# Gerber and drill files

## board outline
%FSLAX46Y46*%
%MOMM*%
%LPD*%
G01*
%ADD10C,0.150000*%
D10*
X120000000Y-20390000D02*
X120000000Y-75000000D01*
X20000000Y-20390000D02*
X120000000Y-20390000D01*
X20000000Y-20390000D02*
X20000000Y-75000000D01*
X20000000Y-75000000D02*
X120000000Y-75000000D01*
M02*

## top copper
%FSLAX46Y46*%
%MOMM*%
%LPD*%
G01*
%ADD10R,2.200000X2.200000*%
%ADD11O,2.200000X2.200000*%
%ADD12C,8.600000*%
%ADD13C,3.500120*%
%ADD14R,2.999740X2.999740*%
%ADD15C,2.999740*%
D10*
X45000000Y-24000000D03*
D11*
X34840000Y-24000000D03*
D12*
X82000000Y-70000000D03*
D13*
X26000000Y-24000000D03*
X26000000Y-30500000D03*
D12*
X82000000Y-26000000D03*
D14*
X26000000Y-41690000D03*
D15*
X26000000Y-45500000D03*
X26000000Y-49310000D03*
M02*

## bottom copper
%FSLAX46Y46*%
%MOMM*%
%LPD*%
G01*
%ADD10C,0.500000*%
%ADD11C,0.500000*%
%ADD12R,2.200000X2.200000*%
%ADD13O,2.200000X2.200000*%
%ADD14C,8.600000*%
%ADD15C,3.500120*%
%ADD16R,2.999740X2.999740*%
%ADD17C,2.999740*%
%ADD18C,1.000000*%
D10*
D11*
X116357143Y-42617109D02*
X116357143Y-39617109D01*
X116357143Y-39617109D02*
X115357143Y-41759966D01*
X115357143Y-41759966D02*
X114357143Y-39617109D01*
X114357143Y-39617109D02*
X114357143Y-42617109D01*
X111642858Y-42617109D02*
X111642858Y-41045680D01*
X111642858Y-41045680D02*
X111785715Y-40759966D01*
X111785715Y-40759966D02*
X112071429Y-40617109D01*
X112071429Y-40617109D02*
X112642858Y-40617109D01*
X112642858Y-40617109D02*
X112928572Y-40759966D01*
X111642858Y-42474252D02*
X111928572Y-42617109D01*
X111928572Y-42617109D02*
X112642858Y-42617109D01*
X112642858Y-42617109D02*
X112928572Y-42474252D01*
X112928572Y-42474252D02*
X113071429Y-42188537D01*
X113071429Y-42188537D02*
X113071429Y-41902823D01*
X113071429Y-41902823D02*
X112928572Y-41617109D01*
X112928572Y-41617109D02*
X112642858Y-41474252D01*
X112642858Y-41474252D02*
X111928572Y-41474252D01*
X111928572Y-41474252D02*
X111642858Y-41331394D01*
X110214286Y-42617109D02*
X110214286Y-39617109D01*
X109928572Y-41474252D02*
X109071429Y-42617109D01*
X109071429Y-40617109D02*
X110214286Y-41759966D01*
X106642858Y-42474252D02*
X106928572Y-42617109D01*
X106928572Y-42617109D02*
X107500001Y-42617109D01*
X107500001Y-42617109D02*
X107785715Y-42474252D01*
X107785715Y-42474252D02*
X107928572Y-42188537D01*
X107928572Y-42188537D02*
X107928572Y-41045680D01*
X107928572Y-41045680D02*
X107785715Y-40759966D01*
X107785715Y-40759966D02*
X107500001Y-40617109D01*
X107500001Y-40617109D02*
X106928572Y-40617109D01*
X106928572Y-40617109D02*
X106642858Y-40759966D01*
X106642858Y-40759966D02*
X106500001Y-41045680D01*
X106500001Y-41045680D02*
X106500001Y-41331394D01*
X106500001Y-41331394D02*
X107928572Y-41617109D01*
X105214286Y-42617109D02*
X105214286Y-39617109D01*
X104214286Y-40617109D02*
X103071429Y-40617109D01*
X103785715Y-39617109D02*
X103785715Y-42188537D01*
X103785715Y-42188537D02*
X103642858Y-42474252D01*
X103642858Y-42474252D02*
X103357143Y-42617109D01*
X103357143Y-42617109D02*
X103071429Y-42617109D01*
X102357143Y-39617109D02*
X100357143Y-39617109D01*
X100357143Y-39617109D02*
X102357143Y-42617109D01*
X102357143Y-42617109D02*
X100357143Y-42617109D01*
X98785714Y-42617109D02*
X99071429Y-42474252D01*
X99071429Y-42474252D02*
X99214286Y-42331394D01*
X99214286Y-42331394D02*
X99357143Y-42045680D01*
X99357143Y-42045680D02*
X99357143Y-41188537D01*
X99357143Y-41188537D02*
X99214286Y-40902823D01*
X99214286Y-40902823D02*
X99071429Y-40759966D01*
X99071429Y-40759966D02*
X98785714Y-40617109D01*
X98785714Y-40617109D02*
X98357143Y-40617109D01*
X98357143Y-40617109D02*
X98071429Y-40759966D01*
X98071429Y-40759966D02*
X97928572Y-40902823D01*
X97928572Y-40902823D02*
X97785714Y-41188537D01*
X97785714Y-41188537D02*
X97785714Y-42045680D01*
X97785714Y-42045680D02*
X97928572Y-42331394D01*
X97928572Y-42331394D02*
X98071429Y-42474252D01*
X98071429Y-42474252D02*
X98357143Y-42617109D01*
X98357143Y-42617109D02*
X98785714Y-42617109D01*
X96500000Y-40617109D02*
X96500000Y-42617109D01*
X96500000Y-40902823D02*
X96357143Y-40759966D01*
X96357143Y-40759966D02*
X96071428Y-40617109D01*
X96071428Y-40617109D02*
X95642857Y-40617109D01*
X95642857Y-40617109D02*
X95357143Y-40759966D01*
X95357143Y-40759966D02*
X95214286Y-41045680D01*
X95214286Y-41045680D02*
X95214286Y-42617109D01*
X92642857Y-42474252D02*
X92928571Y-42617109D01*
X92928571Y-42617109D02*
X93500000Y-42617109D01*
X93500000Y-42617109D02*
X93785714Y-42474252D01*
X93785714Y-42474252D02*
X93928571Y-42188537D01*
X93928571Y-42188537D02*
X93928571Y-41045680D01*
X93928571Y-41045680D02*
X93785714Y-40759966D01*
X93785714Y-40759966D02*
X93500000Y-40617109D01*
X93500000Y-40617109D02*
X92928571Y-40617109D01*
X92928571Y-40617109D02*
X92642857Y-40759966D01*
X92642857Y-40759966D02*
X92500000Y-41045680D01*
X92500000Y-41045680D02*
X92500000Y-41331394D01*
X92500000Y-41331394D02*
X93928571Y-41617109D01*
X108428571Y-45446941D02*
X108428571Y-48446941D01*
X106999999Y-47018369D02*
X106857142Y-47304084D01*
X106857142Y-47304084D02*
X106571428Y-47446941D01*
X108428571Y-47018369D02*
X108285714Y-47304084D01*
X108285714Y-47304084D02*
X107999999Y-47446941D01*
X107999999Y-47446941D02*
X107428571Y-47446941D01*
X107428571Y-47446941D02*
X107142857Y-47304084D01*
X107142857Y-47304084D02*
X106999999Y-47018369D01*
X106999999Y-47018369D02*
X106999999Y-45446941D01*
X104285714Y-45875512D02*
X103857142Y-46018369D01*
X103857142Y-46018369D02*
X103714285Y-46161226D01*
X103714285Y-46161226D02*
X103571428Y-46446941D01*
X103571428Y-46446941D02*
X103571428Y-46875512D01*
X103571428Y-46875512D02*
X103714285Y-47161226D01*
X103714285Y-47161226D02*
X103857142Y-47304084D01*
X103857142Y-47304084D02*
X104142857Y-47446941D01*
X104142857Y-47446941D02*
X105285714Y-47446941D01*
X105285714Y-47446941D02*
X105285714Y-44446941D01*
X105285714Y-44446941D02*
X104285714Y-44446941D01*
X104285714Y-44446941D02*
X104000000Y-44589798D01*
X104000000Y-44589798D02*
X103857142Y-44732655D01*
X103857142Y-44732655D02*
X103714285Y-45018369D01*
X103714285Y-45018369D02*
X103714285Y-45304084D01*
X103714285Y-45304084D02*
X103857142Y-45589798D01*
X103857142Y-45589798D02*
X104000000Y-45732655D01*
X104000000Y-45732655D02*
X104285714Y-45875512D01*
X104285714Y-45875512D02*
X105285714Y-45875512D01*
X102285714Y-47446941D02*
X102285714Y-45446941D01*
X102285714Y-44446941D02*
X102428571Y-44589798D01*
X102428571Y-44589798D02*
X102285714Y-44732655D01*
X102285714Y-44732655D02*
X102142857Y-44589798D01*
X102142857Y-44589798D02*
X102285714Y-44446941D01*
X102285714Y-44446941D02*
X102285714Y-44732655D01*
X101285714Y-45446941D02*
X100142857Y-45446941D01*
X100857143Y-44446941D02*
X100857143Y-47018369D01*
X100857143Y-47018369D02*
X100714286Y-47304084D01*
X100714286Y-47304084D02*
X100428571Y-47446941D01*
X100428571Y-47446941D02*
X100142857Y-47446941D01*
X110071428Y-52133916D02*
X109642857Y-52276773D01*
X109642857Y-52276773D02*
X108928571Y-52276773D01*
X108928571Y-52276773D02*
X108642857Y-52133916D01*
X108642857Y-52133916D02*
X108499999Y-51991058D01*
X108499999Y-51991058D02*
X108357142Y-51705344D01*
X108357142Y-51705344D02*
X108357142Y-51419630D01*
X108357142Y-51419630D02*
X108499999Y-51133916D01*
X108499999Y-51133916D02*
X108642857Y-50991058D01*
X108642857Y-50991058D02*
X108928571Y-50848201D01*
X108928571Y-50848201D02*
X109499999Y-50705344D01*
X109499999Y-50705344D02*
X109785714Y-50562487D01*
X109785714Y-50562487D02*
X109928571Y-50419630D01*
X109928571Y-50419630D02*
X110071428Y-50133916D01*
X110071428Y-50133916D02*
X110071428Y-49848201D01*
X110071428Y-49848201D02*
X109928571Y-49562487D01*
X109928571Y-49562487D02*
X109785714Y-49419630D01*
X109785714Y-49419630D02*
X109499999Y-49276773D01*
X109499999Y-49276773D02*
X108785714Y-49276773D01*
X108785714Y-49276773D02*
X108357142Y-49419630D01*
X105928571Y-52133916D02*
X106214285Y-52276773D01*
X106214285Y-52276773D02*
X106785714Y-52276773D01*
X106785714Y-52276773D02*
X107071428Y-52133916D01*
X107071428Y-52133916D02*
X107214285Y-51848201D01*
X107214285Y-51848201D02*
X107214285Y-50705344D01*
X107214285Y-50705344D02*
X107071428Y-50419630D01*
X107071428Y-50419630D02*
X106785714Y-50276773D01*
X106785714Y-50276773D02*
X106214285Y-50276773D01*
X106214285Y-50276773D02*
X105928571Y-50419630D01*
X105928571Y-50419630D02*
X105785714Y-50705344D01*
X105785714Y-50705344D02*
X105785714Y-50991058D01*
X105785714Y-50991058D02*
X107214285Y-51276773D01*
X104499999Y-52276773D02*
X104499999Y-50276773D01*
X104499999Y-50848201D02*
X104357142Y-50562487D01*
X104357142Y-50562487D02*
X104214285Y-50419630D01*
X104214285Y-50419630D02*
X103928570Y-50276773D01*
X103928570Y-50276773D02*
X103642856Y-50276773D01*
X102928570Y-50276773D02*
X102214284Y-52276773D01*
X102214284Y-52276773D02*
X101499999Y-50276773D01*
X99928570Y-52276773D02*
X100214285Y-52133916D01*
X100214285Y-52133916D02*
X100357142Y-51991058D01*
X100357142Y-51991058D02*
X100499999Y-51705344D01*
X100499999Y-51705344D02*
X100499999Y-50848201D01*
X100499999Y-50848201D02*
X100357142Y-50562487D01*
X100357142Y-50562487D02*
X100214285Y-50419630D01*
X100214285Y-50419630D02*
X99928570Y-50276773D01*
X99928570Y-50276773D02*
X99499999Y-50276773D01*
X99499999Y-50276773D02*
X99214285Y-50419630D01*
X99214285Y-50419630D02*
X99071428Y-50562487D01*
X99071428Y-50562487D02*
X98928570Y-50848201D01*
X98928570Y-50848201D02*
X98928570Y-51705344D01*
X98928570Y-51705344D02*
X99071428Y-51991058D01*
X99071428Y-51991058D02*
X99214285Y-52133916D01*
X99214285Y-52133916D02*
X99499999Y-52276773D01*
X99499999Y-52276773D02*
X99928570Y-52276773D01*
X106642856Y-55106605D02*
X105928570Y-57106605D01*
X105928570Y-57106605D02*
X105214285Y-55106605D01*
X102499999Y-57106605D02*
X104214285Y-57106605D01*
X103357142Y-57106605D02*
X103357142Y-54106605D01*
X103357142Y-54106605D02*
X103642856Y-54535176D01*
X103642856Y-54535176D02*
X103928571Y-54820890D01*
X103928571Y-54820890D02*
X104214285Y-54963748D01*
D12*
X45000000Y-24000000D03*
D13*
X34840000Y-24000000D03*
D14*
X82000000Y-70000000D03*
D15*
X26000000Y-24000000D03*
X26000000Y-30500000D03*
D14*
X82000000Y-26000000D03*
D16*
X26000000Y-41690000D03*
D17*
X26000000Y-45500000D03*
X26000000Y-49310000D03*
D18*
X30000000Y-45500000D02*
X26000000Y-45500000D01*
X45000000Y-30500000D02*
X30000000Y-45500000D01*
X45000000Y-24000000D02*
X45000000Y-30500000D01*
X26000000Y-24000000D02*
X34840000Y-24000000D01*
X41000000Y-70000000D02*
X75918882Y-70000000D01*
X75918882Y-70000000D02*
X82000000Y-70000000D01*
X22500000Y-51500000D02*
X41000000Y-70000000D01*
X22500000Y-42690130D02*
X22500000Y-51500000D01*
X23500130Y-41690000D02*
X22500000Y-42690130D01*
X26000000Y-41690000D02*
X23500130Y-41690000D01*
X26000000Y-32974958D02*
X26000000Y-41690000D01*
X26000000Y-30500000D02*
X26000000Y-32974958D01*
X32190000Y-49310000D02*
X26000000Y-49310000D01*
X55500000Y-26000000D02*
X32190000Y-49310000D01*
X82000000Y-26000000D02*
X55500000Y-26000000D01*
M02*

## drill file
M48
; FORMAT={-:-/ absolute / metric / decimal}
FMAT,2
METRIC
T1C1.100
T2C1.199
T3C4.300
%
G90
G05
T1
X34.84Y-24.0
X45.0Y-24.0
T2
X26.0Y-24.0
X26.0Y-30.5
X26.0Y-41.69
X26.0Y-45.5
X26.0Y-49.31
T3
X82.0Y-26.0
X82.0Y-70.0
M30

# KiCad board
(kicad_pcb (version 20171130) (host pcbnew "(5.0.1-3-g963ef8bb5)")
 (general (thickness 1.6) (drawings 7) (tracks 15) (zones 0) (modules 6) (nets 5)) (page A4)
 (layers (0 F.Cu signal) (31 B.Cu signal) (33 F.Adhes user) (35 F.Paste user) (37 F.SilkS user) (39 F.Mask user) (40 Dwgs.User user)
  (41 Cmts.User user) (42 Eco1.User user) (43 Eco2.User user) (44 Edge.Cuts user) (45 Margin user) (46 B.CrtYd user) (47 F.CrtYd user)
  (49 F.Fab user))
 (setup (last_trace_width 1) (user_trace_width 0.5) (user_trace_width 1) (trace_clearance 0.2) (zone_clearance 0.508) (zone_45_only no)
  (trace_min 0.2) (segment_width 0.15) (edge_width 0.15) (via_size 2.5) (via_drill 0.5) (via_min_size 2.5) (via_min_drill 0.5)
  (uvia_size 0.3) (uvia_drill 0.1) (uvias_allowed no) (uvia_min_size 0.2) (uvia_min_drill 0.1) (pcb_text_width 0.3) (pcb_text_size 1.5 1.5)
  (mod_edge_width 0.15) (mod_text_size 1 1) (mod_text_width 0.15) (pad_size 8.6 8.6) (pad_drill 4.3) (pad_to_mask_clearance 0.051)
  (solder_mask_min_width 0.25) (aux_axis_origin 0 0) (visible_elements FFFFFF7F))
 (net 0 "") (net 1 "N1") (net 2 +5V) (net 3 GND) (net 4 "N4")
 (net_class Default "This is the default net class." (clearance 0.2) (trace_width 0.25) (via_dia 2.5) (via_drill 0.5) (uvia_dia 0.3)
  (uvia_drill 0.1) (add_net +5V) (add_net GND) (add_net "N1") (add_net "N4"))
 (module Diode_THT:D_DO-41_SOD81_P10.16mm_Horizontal (layer F.Cu) (at 45 24 180)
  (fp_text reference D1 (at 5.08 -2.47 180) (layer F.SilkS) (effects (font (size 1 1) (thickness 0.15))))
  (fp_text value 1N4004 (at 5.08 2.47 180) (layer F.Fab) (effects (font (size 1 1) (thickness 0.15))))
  (pad 1 thru_hole rect (at 0 0 180) (size 2.2 2.2) (drill 1.1) (layers *.Cu *.Mask) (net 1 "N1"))
  (pad 2 thru_hole oval (at 10.16 0 180) (size 2.2 2.2) (drill 1.1) (layers *.Cu *.Mask) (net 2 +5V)))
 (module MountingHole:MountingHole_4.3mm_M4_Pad (layer F.Cu) (at 82 70)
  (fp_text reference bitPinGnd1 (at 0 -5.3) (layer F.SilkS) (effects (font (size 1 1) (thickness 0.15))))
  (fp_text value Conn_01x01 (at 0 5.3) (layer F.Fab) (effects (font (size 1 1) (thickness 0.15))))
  (pad 1 thru_hole circle (at 0 0) (size 8.6 8.6) (drill 4.3) (layers *.Cu *.Mask) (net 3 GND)))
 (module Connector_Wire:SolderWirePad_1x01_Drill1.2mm (layer F.Cu) (at 26 24 270)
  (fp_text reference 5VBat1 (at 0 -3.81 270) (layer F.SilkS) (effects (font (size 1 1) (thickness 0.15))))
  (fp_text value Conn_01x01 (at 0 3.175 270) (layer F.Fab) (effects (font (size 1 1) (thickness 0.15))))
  (pad 1 thru_hole circle (at 0 0 270) (size 3.50012 3.50012) (drill 1.19888) (layers *.Cu *.Mask) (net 2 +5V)))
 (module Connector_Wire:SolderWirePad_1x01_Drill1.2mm (layer F.Cu) (at 26 30.5 270)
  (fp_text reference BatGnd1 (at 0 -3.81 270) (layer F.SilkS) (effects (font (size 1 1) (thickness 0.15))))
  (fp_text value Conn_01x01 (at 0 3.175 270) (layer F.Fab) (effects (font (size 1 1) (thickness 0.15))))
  (pad 1 thru_hole circle (at 0 0 270) (size 3.50012 3.50012) (drill 1.19888) (layers *.Cu *.Mask) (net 3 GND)))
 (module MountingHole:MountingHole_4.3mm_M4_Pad (layer F.Cu) (at 82 26)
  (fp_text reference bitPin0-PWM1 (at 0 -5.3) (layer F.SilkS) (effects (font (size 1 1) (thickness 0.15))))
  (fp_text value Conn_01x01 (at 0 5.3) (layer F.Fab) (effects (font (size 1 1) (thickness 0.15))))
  (pad 1 thru_hole circle (at 0 0) (size 8.6 8.6) (drill 4.3) (layers *.Cu *.Mask) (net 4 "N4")))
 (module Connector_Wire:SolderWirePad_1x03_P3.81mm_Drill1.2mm (layer F.Cu) (at 26 41.69 270)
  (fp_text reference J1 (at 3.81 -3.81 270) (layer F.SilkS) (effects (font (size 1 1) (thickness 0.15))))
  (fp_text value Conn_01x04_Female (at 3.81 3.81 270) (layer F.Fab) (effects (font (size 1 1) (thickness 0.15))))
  (pad 1 thru_hole rect (at 0 0 270) (size 2.99974 2.99974) (drill 1.19888) (layers *.Cu *.Mask) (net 3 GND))
  (pad 2 thru_hole circle (at 3.81 0 270) (size 2.99974 2.99974) (drill 1.19888) (layers *.Cu *.Mask) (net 1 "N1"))
  (pad 3 thru_hole circle (at 7.62 0 270) (size 2.99974 2.99974) (drill 1.19888) (layers *.Cu *.Mask) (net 4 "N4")))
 (gr_line (start 120 20.39) (end 120 75) (layer Edge.Cuts) (width 0.15))
 (gr_line (start 20 20.39) (end 120 20.39) (layer Edge.Cuts) (width 0.15))
 (gr_line (start 20 20.39) (end 20 75) (layer Edge.Cuts) (width 0.15))
 (gr_line (start 20 75) (end 120 75) (layer Edge.Cuts) (width 0.15))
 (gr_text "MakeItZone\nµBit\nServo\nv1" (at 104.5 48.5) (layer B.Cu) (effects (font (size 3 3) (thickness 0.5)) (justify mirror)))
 (segment (start 30 45.5) (end 26 45.5) (width 1) (layer B.Cu) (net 1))
 (segment (start 45 30.5) (end 30 45.5) (width 1) (layer B.Cu) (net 1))
 (segment (start 45 24) (end 45 30.5) (width 1) (layer B.Cu) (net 1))
 (segment (start 26 24) (end 34.84 24) (width 1) (layer B.Cu) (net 2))
 (segment (start 41 70) (end 75.918882 70) (width 1) (layer B.Cu) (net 3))
 (segment (start 75.918882 70) (end 82 70) (width 1) (layer B.Cu) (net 3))
 (segment (start 22.5 51.5) (end 41 70) (width 1) (layer B.Cu) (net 3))
 (segment (start 22.5 42.69013) (end 22.5 51.5) (width 1) (layer B.Cu) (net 3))
 (segment (start 23.50013 41.69) (end 22.5 42.69013) (width 1) (layer B.Cu) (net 3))
 (segment (start 26 41.69) (end 23.50013 41.69) (width 1) (layer B.Cu) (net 3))
 (segment (start 26 32.974958) (end 26 41.69) (width 1) (layer B.Cu) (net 3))
 (segment (start 26 30.5) (end 26 32.974958) (width 1) (layer B.Cu) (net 3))
 (segment (start 32.19 49.31) (end 26 49.31) (width 1) (layer B.Cu) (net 4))
 (segment (start 55.5 26) (end 32.19 49.31) (width 1) (layer B.Cu) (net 4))
 (segment (start 82 26) (end 55.5 26) (width 1) (layer B.Cu) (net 4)))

